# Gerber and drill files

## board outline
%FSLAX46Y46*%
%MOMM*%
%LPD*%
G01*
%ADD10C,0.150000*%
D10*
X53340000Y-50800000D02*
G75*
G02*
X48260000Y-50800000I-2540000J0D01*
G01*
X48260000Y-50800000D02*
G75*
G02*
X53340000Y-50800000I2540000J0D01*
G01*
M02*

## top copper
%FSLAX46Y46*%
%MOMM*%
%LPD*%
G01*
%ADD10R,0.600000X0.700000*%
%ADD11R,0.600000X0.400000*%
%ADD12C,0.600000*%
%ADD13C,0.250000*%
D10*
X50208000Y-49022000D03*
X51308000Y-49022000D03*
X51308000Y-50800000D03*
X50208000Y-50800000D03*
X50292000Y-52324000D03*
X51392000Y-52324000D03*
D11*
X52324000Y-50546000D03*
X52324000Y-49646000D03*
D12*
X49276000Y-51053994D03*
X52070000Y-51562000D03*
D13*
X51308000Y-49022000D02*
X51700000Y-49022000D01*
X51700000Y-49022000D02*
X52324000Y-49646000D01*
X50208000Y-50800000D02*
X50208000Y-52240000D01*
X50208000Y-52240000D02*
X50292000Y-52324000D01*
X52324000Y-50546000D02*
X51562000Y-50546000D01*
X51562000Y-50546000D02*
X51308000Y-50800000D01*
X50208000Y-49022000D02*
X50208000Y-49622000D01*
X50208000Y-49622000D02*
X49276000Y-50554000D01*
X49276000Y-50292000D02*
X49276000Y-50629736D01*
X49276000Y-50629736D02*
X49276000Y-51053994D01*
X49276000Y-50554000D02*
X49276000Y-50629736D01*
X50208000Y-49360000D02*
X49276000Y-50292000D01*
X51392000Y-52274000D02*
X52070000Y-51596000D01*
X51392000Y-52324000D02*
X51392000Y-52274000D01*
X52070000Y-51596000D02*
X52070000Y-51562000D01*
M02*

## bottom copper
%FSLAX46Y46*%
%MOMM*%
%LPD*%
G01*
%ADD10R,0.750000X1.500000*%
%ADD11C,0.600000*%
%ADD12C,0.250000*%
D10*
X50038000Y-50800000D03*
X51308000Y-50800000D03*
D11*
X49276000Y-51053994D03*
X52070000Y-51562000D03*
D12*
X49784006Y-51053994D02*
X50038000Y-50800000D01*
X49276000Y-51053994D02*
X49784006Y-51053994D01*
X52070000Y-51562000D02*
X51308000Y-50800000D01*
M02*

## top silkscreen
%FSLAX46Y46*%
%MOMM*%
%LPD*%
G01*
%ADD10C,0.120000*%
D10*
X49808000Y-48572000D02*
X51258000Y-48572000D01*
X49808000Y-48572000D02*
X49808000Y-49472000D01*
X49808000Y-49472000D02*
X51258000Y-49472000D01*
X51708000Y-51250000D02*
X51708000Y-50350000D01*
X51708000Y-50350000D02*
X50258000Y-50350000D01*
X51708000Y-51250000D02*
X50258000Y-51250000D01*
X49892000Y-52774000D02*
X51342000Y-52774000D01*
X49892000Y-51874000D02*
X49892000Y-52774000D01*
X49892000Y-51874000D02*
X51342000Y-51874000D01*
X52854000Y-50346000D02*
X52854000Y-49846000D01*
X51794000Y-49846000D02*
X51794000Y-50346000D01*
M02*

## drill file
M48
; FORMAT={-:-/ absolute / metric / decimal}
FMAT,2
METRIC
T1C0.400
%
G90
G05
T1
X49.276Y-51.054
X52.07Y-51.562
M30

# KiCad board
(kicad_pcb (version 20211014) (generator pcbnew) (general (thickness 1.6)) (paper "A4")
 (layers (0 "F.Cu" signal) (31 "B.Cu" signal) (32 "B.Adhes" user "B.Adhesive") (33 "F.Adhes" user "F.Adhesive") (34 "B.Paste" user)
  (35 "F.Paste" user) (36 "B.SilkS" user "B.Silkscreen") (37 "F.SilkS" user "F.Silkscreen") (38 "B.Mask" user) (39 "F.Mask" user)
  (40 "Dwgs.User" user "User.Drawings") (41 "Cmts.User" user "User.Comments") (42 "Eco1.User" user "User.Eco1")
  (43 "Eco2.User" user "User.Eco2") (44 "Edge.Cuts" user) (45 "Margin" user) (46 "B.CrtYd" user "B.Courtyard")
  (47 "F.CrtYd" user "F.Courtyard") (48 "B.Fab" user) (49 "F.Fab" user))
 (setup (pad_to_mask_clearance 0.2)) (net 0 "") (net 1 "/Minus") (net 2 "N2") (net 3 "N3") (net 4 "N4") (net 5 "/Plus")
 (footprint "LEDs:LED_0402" (layer "F.Cu") (at 50.758 49.022)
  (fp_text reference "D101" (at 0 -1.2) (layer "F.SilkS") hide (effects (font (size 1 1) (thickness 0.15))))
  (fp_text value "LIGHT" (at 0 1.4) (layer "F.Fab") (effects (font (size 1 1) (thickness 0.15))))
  (fp_line (start -0.95 -0.45) (end 0.5 -0.45) (layer "F.SilkS") (width 0.12))
  (fp_line (start -0.95 -0.45) (end -0.95 0.45) (layer "F.SilkS") (width 0.12))
  (fp_line (start -0.95 0.45) (end 0.5 0.45) (layer "F.SilkS") (width 0.12))
  (pad "1" smd rect locked (at -0.55 0 180) (size 0.6 0.7) (layers "F.Cu" "F.Paste" "F.Mask") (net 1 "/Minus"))
  (pad "2" smd rect locked (at 0.55 0 180) (size 0.6 0.7) (layers "F.Cu" "F.Paste" "F.Mask") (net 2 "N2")))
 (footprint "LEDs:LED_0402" (layer "F.Cu") (at 50.758 50.8 180)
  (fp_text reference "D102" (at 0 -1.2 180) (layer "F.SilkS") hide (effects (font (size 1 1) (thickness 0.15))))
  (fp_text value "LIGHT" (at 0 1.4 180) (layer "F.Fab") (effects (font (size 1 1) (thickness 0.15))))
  (fp_line (start -0.95 -0.45) (end -0.95 0.45) (layer "F.SilkS") (width 0.12))
  (fp_line (start -0.95 0.45) (end 0.5 0.45) (layer "F.SilkS") (width 0.12))
  (fp_line (start -0.95 -0.45) (end 0.5 -0.45) (layer "F.SilkS") (width 0.12))
  (pad "1" smd rect locked (at -0.55 0) (size 0.6 0.7) (layers "F.Cu" "F.Paste" "F.Mask") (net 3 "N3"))
  (pad "2" smd rect locked (at 0.55 0) (size 0.6 0.7) (layers "F.Cu" "F.Paste" "F.Mask") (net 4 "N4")))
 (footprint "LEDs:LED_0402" (layer "F.Cu") (at 50.842 52.324)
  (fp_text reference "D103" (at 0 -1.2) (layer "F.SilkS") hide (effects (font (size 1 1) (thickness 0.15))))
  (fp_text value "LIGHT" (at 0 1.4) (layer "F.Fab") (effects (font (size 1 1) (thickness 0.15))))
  (fp_line (start -0.95 0.45) (end 0.5 0.45) (layer "F.SilkS") (width 0.12))
  (fp_line (start -0.95 -0.45) (end -0.95 0.45) (layer "F.SilkS") (width 0.12))
  (fp_line (start -0.95 -0.45) (end 0.5 -0.45) (layer "F.SilkS") (width 0.12))
  (pad "1" smd rect locked (at -0.55 0 180) (size 0.6 0.7) (layers "F.Cu" "F.Paste" "F.Mask") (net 4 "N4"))
  (pad "2" smd rect locked (at 0.55 0 180) (size 0.6 0.7) (layers "F.Cu" "F.Paste" "F.Mask") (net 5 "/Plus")))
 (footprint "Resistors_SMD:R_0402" (layer "F.Cu") (at 52.324 50.096 90)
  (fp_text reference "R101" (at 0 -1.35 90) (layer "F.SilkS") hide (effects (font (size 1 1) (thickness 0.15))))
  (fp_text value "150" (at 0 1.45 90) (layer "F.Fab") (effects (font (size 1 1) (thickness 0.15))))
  (fp_line (start -0.25 0.53) (end 0.25 0.53) (layer "F.SilkS") (width 0.12))
  (fp_line (start 0.25 -0.53) (end -0.25 -0.53) (layer "F.SilkS") (width 0.12))
  (pad "1" smd rect locked (at -0.45 0 90) (size 0.4 0.6) (layers "F.Cu" "F.Paste" "F.Mask") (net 3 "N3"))
  (pad "2" smd rect locked (at 0.45 0 90) (size 0.4 0.6) (layers "F.Cu" "F.Paste" "F.Mask") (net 2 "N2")))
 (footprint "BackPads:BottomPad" (layer "F.Cu") (at 50.038 50.8)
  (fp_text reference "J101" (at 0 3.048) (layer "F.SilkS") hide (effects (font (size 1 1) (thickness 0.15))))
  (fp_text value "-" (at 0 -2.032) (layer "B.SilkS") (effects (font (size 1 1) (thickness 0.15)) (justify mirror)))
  (pad "1" smd rect locked (at 0 0) (size 0.75 1.5) (layers "B.Cu" "B.Paste" "B.Mask") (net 1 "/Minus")))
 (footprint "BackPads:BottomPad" (layer "F.Cu") (at 51.308 50.8)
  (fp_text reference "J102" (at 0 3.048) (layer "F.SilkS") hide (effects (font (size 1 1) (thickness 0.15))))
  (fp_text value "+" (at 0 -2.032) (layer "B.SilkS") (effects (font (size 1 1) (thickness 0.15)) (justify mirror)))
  (pad "1" smd rect locked (at 0 0) (size 0.75 1.5) (layers "B.Cu" "B.Paste" "B.Mask") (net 5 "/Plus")))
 (gr_circle (center 50.8 50.8) (end 53.34 50.8) (layer "Edge.Cuts") (width 0.15) (fill none))
 (segment (start 51.308 49.022) (end 51.7 49.022) (width 0.25) (layer "F.Cu") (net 2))
 (segment (start 51.7 49.022) (end 52.324 49.646) (width 0.25) (layer "F.Cu") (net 2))
 (segment (start 50.208 50.8) (end 50.208 52.24) (width 0.25) (layer "F.Cu") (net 4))
 (segment (start 50.208 52.24) (end 50.292 52.324) (width 0.25) (layer "F.Cu") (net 4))
 (segment (start 52.324 50.546) (end 51.562 50.546) (width 0.25) (layer "F.Cu") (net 3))
 (segment (start 51.562 50.546) (end 51.308 50.8) (width 0.25) (layer "F.Cu") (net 3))
 (segment (start 50.208 49.022) (end 50.208 49.622) (width 0.25) (layer "F.Cu") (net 1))
 (segment (start 50.208 49.622) (end 49.276 50.554) (width 0.25) (layer "F.Cu") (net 1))
 (segment (start 49.276 50.292) (end 49.276 50.629736) (width 0.25) (layer "F.Cu") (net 1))
 (segment (start 49.276 50.629736) (end 49.276 51.053994) (width 0.25) (layer "F.Cu") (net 1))
 (segment (start 49.276 50.554) (end 49.276 50.629736) (width 0.25) (layer "F.Cu") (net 1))
 (segment (start 50.208 49.36) (end 49.276 50.292) (width 0.25) (layer "F.Cu") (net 1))
 (via (at 49.276 51.053994) (size 0.6) (drill 0.4) (layers "F.Cu" "B.Cu") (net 1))
 (segment (start 49.784006 51.053994) (end 50.038 50.8) (width 0.25) (layer "B.Cu") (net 1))
 (segment (start 49.276 51.053994) (end 49.784006 51.053994) (width 0.25) (layer "B.Cu") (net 1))
 (segment (start 51.392 52.274) (end 52.07 51.596) (width 0.25) (layer "F.Cu") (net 5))
 (segment (start 51.392 52.324) (end 51.392 52.274) (width 0.25) (layer "F.Cu") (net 5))
 (segment (start 52.07 51.596) (end 52.07 51.562) (width 0.25) (layer "F.Cu") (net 5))
 (via (at 52.07 51.562) (size 0.6) (drill 0.4) (layers "F.Cu" "B.Cu") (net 5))
 (segment (start 52.07 51.562) (end 51.308 50.8) (width 0.25) (layer "B.Cu") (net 5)))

